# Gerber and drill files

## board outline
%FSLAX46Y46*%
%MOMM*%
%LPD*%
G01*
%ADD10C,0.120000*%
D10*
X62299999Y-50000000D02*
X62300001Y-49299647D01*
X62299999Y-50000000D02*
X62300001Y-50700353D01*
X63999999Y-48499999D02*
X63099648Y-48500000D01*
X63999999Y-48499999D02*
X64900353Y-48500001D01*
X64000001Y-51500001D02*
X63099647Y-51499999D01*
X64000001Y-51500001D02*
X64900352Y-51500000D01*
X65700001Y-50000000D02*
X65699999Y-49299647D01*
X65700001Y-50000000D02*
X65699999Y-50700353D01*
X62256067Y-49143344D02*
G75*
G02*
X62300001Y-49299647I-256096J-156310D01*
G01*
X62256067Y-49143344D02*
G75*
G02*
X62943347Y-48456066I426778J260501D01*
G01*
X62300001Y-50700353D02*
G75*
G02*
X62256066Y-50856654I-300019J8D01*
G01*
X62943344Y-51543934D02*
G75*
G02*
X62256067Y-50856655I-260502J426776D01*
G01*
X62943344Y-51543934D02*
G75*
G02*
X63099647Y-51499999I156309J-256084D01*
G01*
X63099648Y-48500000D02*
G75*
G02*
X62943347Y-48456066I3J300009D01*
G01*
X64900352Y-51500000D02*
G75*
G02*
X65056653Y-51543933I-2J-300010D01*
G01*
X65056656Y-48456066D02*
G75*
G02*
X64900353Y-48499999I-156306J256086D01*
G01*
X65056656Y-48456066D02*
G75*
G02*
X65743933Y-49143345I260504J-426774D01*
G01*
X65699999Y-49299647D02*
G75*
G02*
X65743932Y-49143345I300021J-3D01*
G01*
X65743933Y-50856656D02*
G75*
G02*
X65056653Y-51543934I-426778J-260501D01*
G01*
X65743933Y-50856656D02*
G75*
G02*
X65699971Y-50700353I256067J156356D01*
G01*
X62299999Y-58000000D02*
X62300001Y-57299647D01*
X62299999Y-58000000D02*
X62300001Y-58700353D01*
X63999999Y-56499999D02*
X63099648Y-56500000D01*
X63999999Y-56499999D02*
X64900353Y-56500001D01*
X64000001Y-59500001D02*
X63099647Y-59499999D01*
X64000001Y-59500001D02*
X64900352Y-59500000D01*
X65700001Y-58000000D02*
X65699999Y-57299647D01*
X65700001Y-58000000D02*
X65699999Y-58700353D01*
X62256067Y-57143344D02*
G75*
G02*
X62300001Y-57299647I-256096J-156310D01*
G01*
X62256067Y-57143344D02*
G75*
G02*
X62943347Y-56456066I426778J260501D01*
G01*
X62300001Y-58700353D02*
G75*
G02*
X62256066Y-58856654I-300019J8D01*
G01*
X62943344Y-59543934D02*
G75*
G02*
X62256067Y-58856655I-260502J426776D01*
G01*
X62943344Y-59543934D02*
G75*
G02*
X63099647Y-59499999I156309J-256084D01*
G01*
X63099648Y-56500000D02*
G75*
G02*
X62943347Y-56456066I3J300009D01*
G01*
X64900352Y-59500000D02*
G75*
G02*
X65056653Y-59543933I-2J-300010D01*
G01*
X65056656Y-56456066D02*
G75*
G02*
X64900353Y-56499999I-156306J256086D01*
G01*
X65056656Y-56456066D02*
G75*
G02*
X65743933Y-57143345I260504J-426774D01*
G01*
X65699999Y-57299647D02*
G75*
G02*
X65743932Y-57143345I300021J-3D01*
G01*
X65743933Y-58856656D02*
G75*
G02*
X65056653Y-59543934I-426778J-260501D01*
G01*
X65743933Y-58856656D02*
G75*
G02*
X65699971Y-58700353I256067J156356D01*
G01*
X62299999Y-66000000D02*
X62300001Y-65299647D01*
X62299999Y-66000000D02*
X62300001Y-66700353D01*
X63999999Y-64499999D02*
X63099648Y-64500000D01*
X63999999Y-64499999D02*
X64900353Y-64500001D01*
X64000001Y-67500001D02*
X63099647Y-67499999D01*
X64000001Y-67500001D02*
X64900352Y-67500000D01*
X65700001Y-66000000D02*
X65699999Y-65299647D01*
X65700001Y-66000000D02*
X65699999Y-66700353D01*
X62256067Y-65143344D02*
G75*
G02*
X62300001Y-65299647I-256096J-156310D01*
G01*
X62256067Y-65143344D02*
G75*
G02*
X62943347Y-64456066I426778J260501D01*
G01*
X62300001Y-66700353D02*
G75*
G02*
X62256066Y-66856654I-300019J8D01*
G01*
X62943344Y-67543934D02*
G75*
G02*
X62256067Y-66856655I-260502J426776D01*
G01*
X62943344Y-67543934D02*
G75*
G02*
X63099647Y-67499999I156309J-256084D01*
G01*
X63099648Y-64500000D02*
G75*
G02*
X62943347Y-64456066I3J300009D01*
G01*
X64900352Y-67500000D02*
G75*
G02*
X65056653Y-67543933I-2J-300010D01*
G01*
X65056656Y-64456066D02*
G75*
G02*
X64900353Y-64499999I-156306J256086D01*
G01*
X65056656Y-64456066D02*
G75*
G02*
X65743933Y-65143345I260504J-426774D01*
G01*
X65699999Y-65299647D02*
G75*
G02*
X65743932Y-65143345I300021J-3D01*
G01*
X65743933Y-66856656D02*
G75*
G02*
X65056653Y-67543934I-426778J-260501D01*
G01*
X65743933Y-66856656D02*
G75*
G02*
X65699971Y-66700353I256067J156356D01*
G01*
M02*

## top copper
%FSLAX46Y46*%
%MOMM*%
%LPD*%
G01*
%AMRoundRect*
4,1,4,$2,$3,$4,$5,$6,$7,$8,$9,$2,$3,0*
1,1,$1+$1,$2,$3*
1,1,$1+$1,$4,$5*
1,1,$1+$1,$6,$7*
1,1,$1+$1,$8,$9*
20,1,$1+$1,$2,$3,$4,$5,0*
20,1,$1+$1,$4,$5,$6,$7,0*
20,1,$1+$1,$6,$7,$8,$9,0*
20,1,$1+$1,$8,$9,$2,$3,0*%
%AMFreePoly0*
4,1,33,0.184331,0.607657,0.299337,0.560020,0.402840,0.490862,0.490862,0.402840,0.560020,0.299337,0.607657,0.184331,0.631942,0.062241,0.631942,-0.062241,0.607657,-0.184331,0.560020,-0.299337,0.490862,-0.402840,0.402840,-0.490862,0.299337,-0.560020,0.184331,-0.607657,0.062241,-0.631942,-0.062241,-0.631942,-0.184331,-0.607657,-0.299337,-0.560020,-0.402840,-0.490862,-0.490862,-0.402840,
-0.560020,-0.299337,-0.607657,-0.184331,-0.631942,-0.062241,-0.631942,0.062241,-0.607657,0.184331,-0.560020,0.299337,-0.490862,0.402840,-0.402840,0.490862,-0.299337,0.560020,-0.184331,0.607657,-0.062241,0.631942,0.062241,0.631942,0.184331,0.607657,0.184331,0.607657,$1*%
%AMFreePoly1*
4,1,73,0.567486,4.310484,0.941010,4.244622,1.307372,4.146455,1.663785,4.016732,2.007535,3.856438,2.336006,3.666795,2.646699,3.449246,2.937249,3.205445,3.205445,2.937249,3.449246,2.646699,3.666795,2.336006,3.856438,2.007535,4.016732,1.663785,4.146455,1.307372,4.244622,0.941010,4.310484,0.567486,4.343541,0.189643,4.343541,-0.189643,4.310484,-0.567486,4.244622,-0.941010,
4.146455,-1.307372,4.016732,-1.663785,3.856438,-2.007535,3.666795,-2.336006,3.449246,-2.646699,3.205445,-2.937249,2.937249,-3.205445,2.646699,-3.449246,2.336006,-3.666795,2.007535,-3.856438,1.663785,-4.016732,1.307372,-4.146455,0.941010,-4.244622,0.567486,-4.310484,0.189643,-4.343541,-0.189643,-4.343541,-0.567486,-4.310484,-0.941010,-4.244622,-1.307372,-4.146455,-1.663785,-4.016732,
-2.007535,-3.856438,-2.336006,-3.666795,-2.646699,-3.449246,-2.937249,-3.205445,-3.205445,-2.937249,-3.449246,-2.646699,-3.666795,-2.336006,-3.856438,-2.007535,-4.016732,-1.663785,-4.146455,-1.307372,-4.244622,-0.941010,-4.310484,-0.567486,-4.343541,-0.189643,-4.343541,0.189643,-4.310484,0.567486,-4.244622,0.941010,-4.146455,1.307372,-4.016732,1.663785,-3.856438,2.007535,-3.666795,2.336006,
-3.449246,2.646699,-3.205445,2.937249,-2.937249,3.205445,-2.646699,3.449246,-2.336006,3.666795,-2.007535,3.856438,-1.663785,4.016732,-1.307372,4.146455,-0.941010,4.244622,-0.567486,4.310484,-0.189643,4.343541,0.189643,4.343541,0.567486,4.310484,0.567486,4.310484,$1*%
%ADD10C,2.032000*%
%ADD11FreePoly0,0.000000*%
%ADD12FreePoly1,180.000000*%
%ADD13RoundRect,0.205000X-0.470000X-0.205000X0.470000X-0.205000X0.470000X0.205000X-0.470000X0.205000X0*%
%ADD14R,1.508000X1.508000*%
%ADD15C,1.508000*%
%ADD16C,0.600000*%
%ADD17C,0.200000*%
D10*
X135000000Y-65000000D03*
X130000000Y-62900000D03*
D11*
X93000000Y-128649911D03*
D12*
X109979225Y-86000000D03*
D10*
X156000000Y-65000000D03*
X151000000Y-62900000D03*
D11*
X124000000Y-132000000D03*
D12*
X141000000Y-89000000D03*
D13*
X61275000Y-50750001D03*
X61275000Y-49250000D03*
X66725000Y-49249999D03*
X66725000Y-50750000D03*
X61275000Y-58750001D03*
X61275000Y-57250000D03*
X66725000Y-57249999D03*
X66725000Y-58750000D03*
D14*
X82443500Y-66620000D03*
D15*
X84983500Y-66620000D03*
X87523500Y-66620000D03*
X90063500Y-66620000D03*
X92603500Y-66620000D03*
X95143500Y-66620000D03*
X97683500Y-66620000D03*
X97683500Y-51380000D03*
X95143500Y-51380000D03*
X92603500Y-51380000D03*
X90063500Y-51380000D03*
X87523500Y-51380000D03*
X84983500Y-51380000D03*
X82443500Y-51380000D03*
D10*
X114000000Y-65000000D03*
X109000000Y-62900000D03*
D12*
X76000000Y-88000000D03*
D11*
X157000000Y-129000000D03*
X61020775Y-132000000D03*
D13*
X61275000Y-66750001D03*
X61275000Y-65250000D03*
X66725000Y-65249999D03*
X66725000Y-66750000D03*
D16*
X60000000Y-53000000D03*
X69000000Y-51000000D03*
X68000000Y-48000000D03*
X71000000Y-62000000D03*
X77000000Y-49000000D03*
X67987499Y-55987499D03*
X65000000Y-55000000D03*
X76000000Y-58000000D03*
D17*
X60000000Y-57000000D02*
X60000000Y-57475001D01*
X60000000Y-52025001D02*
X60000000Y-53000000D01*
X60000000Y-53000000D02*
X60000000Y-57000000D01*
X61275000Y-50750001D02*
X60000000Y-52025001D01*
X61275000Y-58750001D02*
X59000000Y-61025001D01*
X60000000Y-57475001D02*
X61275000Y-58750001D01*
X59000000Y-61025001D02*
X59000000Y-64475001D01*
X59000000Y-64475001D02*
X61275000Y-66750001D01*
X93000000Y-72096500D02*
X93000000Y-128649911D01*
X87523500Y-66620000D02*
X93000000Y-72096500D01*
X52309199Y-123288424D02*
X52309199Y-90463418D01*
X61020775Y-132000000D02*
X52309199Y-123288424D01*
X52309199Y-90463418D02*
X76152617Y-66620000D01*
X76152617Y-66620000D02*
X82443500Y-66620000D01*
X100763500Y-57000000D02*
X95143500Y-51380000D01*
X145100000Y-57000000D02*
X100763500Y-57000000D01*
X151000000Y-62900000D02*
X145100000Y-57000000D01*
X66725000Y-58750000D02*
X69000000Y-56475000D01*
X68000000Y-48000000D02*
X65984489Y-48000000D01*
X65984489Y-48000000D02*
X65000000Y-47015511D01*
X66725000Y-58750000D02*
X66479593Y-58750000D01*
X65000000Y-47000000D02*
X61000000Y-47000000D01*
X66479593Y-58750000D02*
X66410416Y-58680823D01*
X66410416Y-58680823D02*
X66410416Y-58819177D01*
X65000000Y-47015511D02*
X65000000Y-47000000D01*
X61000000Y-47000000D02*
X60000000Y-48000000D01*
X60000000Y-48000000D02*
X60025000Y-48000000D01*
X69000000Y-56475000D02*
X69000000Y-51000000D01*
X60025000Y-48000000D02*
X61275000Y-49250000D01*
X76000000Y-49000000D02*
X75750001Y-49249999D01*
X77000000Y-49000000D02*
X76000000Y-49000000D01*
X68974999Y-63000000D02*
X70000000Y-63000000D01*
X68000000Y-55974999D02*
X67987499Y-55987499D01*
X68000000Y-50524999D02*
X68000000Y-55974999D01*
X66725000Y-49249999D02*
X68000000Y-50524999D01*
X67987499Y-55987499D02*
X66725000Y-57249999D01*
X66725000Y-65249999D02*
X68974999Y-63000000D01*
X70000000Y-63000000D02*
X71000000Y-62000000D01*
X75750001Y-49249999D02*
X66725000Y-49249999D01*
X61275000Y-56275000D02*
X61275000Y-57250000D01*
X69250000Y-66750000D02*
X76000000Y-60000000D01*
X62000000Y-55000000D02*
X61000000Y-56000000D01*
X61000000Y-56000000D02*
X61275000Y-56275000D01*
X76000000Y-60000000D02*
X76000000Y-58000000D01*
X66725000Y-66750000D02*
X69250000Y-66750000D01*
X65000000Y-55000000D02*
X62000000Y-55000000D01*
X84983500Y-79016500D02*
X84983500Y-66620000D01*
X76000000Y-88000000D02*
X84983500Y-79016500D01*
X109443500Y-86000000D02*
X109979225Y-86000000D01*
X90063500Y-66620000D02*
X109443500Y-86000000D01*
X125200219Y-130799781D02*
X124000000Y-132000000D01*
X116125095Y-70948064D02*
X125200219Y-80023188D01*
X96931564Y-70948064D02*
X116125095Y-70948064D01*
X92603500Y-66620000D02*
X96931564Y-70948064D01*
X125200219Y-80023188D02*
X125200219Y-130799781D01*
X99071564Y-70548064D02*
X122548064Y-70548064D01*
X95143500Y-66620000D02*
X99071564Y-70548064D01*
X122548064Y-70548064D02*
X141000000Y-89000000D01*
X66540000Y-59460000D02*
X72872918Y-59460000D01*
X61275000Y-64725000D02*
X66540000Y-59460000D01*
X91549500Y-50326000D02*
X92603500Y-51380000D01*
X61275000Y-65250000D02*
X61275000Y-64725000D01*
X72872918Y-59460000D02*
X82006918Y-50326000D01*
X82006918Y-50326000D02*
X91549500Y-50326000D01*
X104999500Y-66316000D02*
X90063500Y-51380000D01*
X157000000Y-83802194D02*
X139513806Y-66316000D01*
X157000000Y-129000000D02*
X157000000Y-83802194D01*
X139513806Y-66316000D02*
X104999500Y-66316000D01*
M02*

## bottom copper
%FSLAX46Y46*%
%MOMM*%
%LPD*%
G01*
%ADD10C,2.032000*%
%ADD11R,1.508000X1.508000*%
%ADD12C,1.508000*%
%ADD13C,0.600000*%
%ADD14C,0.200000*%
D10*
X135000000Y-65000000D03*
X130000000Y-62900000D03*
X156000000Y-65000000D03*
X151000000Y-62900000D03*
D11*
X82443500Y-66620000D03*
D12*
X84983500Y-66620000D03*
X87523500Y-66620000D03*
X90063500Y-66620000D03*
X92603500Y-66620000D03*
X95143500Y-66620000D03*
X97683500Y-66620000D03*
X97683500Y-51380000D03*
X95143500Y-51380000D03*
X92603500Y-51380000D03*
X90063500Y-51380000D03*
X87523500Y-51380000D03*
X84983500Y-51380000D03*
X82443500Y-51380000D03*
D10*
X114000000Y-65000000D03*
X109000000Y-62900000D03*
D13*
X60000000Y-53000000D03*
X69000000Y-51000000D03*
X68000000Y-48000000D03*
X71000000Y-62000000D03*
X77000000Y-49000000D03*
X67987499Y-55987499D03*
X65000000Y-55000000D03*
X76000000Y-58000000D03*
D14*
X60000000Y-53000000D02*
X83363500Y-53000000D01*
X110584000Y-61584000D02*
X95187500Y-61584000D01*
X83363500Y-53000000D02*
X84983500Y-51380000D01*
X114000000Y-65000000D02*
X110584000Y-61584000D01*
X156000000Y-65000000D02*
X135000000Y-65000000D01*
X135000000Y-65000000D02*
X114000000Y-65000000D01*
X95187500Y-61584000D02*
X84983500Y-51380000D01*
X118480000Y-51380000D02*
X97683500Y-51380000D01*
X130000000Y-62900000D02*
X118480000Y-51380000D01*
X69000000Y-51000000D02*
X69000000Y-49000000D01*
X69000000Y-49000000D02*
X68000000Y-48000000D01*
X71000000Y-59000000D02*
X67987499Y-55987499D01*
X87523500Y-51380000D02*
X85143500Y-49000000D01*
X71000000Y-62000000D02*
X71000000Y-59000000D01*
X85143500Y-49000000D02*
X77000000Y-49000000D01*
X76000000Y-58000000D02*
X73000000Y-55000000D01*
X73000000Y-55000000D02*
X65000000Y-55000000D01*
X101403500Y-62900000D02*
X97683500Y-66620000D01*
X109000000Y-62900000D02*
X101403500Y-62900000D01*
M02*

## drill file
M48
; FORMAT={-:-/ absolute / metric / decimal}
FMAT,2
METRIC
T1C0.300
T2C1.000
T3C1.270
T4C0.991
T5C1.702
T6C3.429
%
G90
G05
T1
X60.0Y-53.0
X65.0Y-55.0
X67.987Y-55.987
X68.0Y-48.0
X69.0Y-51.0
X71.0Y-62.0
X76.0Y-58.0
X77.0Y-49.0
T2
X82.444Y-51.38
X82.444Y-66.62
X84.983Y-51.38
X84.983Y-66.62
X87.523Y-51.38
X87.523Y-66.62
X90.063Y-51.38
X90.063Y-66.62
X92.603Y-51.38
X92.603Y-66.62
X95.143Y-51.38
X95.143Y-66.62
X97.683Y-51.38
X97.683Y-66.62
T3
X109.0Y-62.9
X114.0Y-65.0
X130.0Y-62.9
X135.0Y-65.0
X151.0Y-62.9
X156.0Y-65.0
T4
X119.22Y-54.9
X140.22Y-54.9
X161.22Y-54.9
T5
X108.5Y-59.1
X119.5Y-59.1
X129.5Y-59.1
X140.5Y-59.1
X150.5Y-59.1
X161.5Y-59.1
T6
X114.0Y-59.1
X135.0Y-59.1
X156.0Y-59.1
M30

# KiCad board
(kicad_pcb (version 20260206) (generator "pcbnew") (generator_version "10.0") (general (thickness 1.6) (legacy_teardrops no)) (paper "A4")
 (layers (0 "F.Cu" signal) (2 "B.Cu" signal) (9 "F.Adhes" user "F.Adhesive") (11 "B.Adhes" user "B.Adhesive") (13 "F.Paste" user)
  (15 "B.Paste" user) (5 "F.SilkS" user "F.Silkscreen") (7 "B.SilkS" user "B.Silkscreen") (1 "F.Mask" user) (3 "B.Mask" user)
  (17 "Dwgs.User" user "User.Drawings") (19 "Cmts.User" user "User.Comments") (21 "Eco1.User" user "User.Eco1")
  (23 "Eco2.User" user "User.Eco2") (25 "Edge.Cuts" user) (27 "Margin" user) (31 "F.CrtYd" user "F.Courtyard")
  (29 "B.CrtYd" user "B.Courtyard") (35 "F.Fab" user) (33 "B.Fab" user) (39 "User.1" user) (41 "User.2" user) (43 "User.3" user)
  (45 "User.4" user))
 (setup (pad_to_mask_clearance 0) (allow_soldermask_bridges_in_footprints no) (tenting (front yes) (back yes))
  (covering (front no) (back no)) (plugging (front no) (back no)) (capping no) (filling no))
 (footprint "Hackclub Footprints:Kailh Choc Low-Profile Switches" (layer "F.Cu") (at 135 59.100001)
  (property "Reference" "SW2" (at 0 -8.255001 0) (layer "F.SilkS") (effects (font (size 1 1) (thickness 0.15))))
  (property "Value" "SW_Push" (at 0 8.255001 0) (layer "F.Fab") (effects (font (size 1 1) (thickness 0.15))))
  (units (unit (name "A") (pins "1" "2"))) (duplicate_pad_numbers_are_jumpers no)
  (pad "" np_thru_hole circle (at -5.5 0) (size 1.7018 1.7018) (drill 1.7018) (layers "*.Cu" "*.Mask"))
  (pad "" np_thru_hole circle (at 0 0) (size 3.429 3.429) (drill 3.429) (layers "*.Cu" "*.Mask"))
  (pad "" np_thru_hole circle (at 5.22 -4.2) (size 0.9906 0.9906) (drill 0.9906) (layers "*.Cu" "*.Mask"))
  (pad "" np_thru_hole circle (at 5.5 0) (size 1.7018 1.7018) (drill 1.7018) (layers "*.Cu" "*.Mask"))
  (pad "1" thru_hole circle (at 0 5.899999) (size 2.032 2.032) (drill 1.27) (layers "*.Cu" "*.Mask") (remove_unused_layers no) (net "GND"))
  (pad "2" thru_hole circle (at -5 3.799999) (size 2.032 2.032) (drill 1.27) (layers "*.Cu" "*.Mask") (remove_unused_layers no)
   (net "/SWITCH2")))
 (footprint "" (layer "F.Cu") (at 93 128.649911)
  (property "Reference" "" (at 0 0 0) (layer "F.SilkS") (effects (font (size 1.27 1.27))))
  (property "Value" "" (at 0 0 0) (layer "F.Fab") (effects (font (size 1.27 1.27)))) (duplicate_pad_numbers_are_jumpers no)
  (pad "3" smd custom (at 0 0) (size 1.27 1.27) (layers "F.Cu" "F.Mask") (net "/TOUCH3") (thermal_bridge_angle 90)
   (options (clearance outline) (anchor circle)) (primitives)))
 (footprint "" (layer "F.Cu") (at 109.979225 86)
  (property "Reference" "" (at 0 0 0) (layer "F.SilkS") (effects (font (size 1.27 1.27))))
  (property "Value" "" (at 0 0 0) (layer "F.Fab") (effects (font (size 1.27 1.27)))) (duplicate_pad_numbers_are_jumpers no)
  (pad "4" smd custom (at 0 0 180) (size 8.695358 8.695358) (layers "F.Cu" "F.Mask") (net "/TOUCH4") (thermal_bridge_angle 90)
   (options (clearance outline) (anchor circle)) (primitives)))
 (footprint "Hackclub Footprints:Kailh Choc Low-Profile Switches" (layer "F.Cu") (at 156 59.100001)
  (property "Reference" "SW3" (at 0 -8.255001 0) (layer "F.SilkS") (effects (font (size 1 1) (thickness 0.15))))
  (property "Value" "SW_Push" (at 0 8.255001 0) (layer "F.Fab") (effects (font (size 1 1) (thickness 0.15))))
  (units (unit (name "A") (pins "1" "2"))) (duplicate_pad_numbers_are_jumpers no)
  (pad "" np_thru_hole circle (at -5.5 0) (size 1.7018 1.7018) (drill 1.7018) (layers "*.Cu" "*.Mask"))
  (pad "" np_thru_hole circle (at 0 0) (size 3.429 3.429) (drill 3.429) (layers "*.Cu" "*.Mask"))
  (pad "" np_thru_hole circle (at 5.22 -4.2) (size 0.9906 0.9906) (drill 0.9906) (layers "*.Cu" "*.Mask"))
  (pad "" np_thru_hole circle (at 5.5 0) (size 1.7018 1.7018) (drill 1.7018) (layers "*.Cu" "*.Mask"))
  (pad "1" thru_hole circle (at 0 5.899999) (size 2.032 2.032) (drill 1.27) (layers "*.Cu" "*.Mask") (remove_unused_layers no) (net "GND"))
  (pad "2" thru_hole circle (at -5 3.799999) (size 2.032 2.032) (drill 1.27) (layers "*.Cu" "*.Mask") (remove_unused_layers no)
   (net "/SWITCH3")))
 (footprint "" (layer "F.Cu") (at 124 132)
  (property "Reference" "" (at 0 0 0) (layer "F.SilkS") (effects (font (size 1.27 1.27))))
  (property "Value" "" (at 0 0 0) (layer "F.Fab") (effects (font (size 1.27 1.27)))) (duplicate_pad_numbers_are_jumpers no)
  (pad "5" smd custom (at 0 0) (size 1.27 1.27) (layers "F.Cu" "F.Mask") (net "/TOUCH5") (thermal_bridge_angle 90)
   (options (clearance outline) (anchor circle)) (primitives)))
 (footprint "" (layer "F.Cu") (at 141 89)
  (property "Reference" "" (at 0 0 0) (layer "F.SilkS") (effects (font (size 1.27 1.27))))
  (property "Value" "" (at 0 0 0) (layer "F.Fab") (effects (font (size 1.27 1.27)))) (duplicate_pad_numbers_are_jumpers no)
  (pad "6" smd custom (at 0 0 180) (size 8.695358 8.695358) (layers "F.Cu" "F.Mask") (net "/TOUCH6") (thermal_bridge_angle 90)
   (options (clearance outline) (anchor circle)) (primitives)))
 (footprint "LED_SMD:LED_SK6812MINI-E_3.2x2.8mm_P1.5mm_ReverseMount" (layer "F.Cu") (at 64 50)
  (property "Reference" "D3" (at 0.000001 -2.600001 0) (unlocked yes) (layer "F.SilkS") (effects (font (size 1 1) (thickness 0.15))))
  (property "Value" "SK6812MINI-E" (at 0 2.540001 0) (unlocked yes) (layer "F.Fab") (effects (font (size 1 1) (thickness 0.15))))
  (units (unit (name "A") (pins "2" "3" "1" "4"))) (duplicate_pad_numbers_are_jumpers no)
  (fp_line (start -1.700001 0) (end -1.699999 -0.700353) (stroke (width 0.12) (type solid)) (layer "Edge.Cuts"))
  (fp_line (start -1.700001 0) (end -1.699999 0.700353) (stroke (width 0.12) (type solid)) (layer "Edge.Cuts"))
  (fp_line (start -0.000001 -1.500001) (end -0.900352 -1.5) (stroke (width 0.12) (type solid)) (layer "Edge.Cuts"))
  (fp_line (start -0.000001 -1.500001) (end 0.900353 -1.499999) (stroke (width 0.12) (type solid)) (layer "Edge.Cuts"))
  (fp_line (start 0.000001 1.500001) (end -0.900353 1.499999) (stroke (width 0.12) (type solid)) (layer "Edge.Cuts"))
  (fp_line (start 0.000001 1.500001) (end 0.900352 1.5) (stroke (width 0.12) (type solid)) (layer "Edge.Cuts"))
  (fp_line (start 1.700001 0) (end 1.699999 -0.700353) (stroke (width 0.12) (type solid)) (layer "Edge.Cuts"))
  (fp_line (start 1.700001 0) (end 1.699999 0.700353) (stroke (width 0.12) (type solid)) (layer "Edge.Cuts"))
  (fp_arc (start -1.743933 -0.856656) (mid -1.711192 -0.781532) (end -1.699999 -0.700353) (stroke (width 0.12) (type solid))
   (layer "Edge.Cuts"))
  (fp_arc (start -1.743933 -0.856656) (mid -1.670709 -1.47071) (end -1.056653 -1.543934) (stroke (width 0.12) (type solid))
   (layer "Edge.Cuts"))
  (fp_arc (start -1.699999 0.700353) (mid -1.711192 0.78153) (end -1.743934 0.856654) (stroke (width 0.12) (type solid)) (layer "Edge.Cuts"))
  (fp_arc (start -1.056656 1.543934) (mid -1.670711 1.470711) (end -1.743934 0.856654) (stroke (width 0.12) (type solid))
   (layer "Edge.Cuts"))
  (fp_arc (start -1.056656 1.543934) (mid -0.981532 1.511192) (end -0.900353 1.499999) (stroke (width 0.12) (type solid))
   (layer "Edge.Cuts"))
  (fp_arc (start -0.900352 -1.5) (mid -0.981532 -1.511193) (end -1.056653 -1.543934) (stroke (width 0.12) (type solid)) (layer "Edge.Cuts"))
  (fp_arc (start 0.900352 1.5) (mid 0.981532 1.511193) (end 1.056653 1.543934) (stroke (width 0.12) (type solid)) (layer "Edge.Cuts"))
  (fp_arc (start 1.056656 -1.543934) (mid 0.981532 -1.511192) (end 0.900353 -1.499999) (stroke (width 0.12) (type solid))
   (layer "Edge.Cuts"))
  (fp_arc (start 1.056656 -1.543934) (mid 1.670711 -1.470711) (end 1.743934 -0.856654) (stroke (width 0.12) (type solid))
   (layer "Edge.Cuts"))
  (fp_arc (start 1.699999 -0.700353) (mid 1.711192 -0.78153) (end 1.743934 -0.856654) (stroke (width 0.12) (type solid)) (layer "Edge.Cuts"))
  (fp_arc (start 1.743933 0.856656) (mid 1.670709 1.47071) (end 1.056653 1.543934) (stroke (width 0.12) (type solid)) (layer "Edge.Cuts"))
  (fp_arc (start 1.743933 0.856656) (mid 1.711192 0.781532) (end 1.699999 0.700353) (stroke (width 0.12) (type solid)) (layer "Edge.Cuts"))
  (pad "1" smd roundrect (at -2.725 0.750001) (size 1.35 0.82) (layers "F.Cu" "F.Mask" "F.Paste") (roundrect_rratio 0.25) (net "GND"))
  (pad "2" smd roundrect (at -2.725 -0.75) (size 1.35 0.82) (layers "F.Cu" "F.Mask" "F.Paste") (roundrect_rratio 0.25) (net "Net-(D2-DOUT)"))
  (pad "3" smd roundrect (at 2.725 -0.750001) (size 1.35 0.82) (layers "F.Cu" "F.Mask" "F.Paste") (roundrect_rratio 0.25) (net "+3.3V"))
  (pad "4" smd roundrect (at 2.725 0.75) (size 1.35 0.82) (layers "F.Cu" "F.Mask" "F.Paste") (roundrect_rratio 0.25)
   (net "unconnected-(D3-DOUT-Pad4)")))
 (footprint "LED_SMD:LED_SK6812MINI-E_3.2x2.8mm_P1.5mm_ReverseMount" (layer "F.Cu") (at 64 58)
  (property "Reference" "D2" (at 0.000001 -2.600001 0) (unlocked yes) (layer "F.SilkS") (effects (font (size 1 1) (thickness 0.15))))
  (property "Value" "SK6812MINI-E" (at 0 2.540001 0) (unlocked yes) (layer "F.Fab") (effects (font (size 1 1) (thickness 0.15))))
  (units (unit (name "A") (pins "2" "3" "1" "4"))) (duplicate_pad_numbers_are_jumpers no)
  (fp_line (start -1.700001 0) (end -1.699999 -0.700353) (stroke (width 0.12) (type solid)) (layer "Edge.Cuts"))
  (fp_line (start -1.700001 0) (end -1.699999 0.700353) (stroke (width 0.12) (type solid)) (layer "Edge.Cuts"))
  (fp_line (start -0.000001 -1.500001) (end -0.900352 -1.5) (stroke (width 0.12) (type solid)) (layer "Edge.Cuts"))
  (fp_line (start -0.000001 -1.500001) (end 0.900353 -1.499999) (stroke (width 0.12) (type solid)) (layer "Edge.Cuts"))
  (fp_line (start 0.000001 1.500001) (end -0.900353 1.499999) (stroke (width 0.12) (type solid)) (layer "Edge.Cuts"))
  (fp_line (start 0.000001 1.500001) (end 0.900352 1.5) (stroke (width 0.12) (type solid)) (layer "Edge.Cuts"))
  (fp_line (start 1.700001 0) (end 1.699999 -0.700353) (stroke (width 0.12) (type solid)) (layer "Edge.Cuts"))
  (fp_line (start 1.700001 0) (end 1.699999 0.700353) (stroke (width 0.12) (type solid)) (layer "Edge.Cuts"))
  (fp_arc (start -1.743933 -0.856656) (mid -1.711192 -0.781532) (end -1.699999 -0.700353) (stroke (width 0.12) (type solid))
   (layer "Edge.Cuts"))
  (fp_arc (start -1.743933 -0.856656) (mid -1.670709 -1.47071) (end -1.056653 -1.543934) (stroke (width 0.12) (type solid))
   (layer "Edge.Cuts"))
  (fp_arc (start -1.699999 0.700353) (mid -1.711192 0.78153) (end -1.743934 0.856654) (stroke (width 0.12) (type solid)) (layer "Edge.Cuts"))
  (fp_arc (start -1.056656 1.543934) (mid -1.670711 1.470711) (end -1.743934 0.856654) (stroke (width 0.12) (type solid))
   (layer "Edge.Cuts"))
  (fp_arc (start -1.056656 1.543934) (mid -0.981532 1.511192) (end -0.900353 1.499999) (stroke (width 0.12) (type solid))
   (layer "Edge.Cuts"))
  (fp_arc (start -0.900352 -1.5) (mid -0.981532 -1.511193) (end -1.056653 -1.543934) (stroke (width 0.12) (type solid)) (layer "Edge.Cuts"))
  (fp_arc (start 0.900352 1.5) (mid 0.981532 1.511193) (end 1.056653 1.543934) (stroke (width 0.12) (type solid)) (layer "Edge.Cuts"))
  (fp_arc (start 1.056656 -1.543934) (mid 0.981532 -1.511192) (end 0.900353 -1.499999) (stroke (width 0.12) (type solid))
   (layer "Edge.Cuts"))
  (fp_arc (start 1.056656 -1.543934) (mid 1.670711 -1.470711) (end 1.743934 -0.856654) (stroke (width 0.12) (type solid))
   (layer "Edge.Cuts"))
  (fp_arc (start 1.699999 -0.700353) (mid 1.711192 -0.78153) (end 1.743934 -0.856654) (stroke (width 0.12) (type solid)) (layer "Edge.Cuts"))
  (fp_arc (start 1.743933 0.856656) (mid 1.670709 1.47071) (end 1.056653 1.543934) (stroke (width 0.12) (type solid)) (layer "Edge.Cuts"))
  (fp_arc (start 1.743933 0.856656) (mid 1.711192 0.781532) (end 1.699999 0.700353) (stroke (width 0.12) (type solid)) (layer "Edge.Cuts"))
  (pad "1" smd roundrect (at -2.725 0.750001) (size 1.35 0.82) (layers "F.Cu" "F.Mask" "F.Paste") (roundrect_rratio 0.25) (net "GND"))
  (pad "2" smd roundrect (at -2.725 -0.75) (size 1.35 0.82) (layers "F.Cu" "F.Mask" "F.Paste") (roundrect_rratio 0.25) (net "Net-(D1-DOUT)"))
  (pad "3" smd roundrect (at 2.725 -0.750001) (size 1.35 0.82) (layers "F.Cu" "F.Mask" "F.Paste") (roundrect_rratio 0.25) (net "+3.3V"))
  (pad "4" smd roundrect (at 2.725 0.75) (size 1.35 0.82) (layers "F.Cu" "F.Mask" "F.Paste") (roundrect_rratio 0.25) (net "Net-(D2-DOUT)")))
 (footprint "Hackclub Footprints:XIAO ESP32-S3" (layer "F.Cu") (at 90 59 90)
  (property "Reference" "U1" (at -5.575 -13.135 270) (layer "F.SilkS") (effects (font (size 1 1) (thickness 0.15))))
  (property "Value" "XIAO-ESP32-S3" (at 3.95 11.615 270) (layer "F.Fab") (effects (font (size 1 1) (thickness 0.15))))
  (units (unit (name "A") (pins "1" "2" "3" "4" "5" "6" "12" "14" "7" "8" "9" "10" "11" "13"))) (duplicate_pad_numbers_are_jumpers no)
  (pad "1" thru_hole rect (at -7.62 -7.5565 90) (size 1.508 1.508) (drill 1) (layers "*.Cu" "*.Mask") (remove_unused_layers no)
   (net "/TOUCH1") (solder_mask_margin 0.102))
  (pad "2" thru_hole circle (at -7.62 -5.0165 90) (size 1.508 1.508) (drill 1) (layers "*.Cu" "*.Mask") (remove_unused_layers no)
   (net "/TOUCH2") (solder_mask_margin 0.102))
  (pad "3" thru_hole circle (at -7.62 -2.4765 90) (size 1.508 1.508) (drill 1) (layers "*.Cu" "*.Mask") (remove_unused_layers no)
   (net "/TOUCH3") (solder_mask_margin 0.102))
  (pad "4" thru_hole circle (at -7.62 0.0635 90) (size 1.508 1.508) (drill 1) (layers "*.Cu" "*.Mask") (remove_unused_layers no)
   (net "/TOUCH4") (solder_mask_margin 0.102))
  (pad "5" thru_hole circle (at -7.62 2.6035 90) (size 1.508 1.508) (drill 1) (layers "*.Cu" "*.Mask") (remove_unused_layers no)
   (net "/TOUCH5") (solder_mask_margin 0.102))
  (pad "6" thru_hole circle (at -7.62 5.1435 90) (size 1.508 1.508) (drill 1) (layers "*.Cu" "*.Mask") (remove_unused_layers no)
   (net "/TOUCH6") (solder_mask_margin 0.102))
  (pad "7" thru_hole circle (at -7.62 7.6835 90) (size 1.508 1.508) (drill 1) (layers "*.Cu" "*.Mask") (remove_unused_layers no)
   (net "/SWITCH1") (solder_mask_margin 0.102))
  (pad "8" thru_hole circle (at 7.62 7.6835 90) (size 1.508 1.508) (drill 1) (layers "*.Cu" "*.Mask") (remove_unused_layers no)
   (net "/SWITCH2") (solder_mask_margin 0.102))
  (pad "9" thru_hole circle (at 7.62 5.1435 90) (size 1.508 1.508) (drill 1) (layers "*.Cu" "*.Mask") (remove_unused_layers no)
   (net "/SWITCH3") (solder_mask_margin 0.102))
  (pad "10" thru_hole circle (at 7.62 2.6035 90) (size 1.508 1.508) (drill 1) (layers "*.Cu" "*.Mask") (remove_unused_layers no)
   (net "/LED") (solder_mask_margin 0.102))
  (pad "11" thru_hole circle (at 7.62 0.0635 90) (size 1.508 1.508) (drill 1) (layers "*.Cu" "*.Mask") (remove_unused_layers no)
   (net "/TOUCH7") (solder_mask_margin 0.102))
  (pad "12" thru_hole circle (at 7.62 -2.4765 90) (size 1.508 1.508) (drill 1) (layers "*.Cu" "*.Mask") (remove_unused_layers no)
   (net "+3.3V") (solder_mask_margin 0.102))
  (pad "13" thru_hole circle (at 7.62 -5.0165 90) (size 1.508 1.508) (drill 1) (layers "*.Cu" "*.Mask") (remove_unused_layers no)
   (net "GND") (solder_mask_margin 0.102))
  (pad "14" thru_hole circle (at 7.62 -7.5565 90) (size 1.508 1.508) (drill 1) (layers "*.Cu" "*.Mask") (remove_unused_layers no)
   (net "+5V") (solder_mask_margin 0.102)))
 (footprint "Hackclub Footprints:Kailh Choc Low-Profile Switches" (layer "F.Cu") (at 114 59.100001)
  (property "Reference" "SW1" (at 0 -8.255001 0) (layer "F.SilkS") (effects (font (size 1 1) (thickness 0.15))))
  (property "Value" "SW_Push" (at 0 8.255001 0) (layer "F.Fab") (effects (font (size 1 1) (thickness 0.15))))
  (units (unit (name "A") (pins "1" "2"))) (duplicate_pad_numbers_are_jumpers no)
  (pad "" np_thru_hole circle (at -5.5 0) (size 1.7018 1.7018) (drill 1.7018) (layers "*.Cu" "*.Mask"))
  (pad "" np_thru_hole circle (at 0 0) (size 3.429 3.429) (drill 3.429) (layers "*.Cu" "*.Mask"))
  (pad "" np_thru_hole circle (at 5.22 -4.2) (size 0.9906 0.9906) (drill 0.9906) (layers "*.Cu" "*.Mask"))
  (pad "" np_thru_hole circle (at 5.5 0) (size 1.7018 1.7018) (drill 1.7018) (layers "*.Cu" "*.Mask"))
  (pad "1" thru_hole circle (at 0 5.899999) (size 2.032 2.032) (drill 1.27) (layers "*.Cu" "*.Mask") (remove_unused_layers no) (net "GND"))
  (pad "2" thru_hole circle (at -5 3.799999) (size 2.032 2.032) (drill 1.27) (layers "*.Cu" "*.Mask") (remove_unused_layers no)
   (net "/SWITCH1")))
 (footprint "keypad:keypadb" (layer "F.Cu") (at 76 103.301057 180)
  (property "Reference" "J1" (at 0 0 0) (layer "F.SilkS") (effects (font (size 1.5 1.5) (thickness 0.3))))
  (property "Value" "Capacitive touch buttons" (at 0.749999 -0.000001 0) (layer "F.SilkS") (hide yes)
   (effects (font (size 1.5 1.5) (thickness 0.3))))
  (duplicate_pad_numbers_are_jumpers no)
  (pad "2" smd custom (at 0 15.301057 180) (size 8.695358 8.695358) (layers "F.Cu" "F.Mask") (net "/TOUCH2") (thermal_bridge_angle 90)
   (options (clearance outline) (anchor circle)) (primitives)))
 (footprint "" (layer "F.Cu") (at 157 129)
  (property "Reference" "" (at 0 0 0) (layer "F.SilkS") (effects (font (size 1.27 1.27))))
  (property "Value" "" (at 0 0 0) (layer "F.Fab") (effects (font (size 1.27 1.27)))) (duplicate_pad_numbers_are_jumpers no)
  (pad "7" smd custom (at 0 0) (size 1.27 1.27) (layers "F.Cu" "F.Mask") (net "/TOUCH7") (thermal_bridge_angle 90)
   (options (clearance outline) (anchor circle)) (primitives)))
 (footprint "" (layer "F.Cu") (at 61.020775 132)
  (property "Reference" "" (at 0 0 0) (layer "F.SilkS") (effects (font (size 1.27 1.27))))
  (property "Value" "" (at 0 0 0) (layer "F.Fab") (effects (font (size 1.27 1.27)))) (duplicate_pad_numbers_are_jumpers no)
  (pad "1" smd custom (at 0 0) (size 1.27 1.27) (layers "F.Cu" "F.Mask") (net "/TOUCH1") (thermal_bridge_angle 90)
   (options (clearance outline) (anchor circle)) (primitives)))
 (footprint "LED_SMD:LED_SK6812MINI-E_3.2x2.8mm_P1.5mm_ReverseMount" (layer "F.Cu") (at 64 66)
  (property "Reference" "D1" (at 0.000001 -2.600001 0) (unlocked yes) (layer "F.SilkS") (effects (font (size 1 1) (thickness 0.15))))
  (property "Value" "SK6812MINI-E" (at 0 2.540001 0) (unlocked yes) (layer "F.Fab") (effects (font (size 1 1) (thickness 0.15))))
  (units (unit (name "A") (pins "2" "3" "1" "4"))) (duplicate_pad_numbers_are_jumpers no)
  (fp_line (start -1.700001 0) (end -1.699999 -0.700353) (stroke (width 0.12) (type solid)) (layer "Edge.Cuts"))
  (fp_line (start -1.700001 0) (end -1.699999 0.700353) (stroke (width 0.12) (type solid)) (layer "Edge.Cuts"))
  (fp_line (start -0.000001 -1.500001) (end -0.900352 -1.5) (stroke (width 0.12) (type solid)) (layer "Edge.Cuts"))
  (fp_line (start -0.000001 -1.500001) (end 0.900353 -1.499999) (stroke (width 0.12) (type solid)) (layer "Edge.Cuts"))
  (fp_line (start 0.000001 1.500001) (end -0.900353 1.499999) (stroke (width 0.12) (type solid)) (layer "Edge.Cuts"))
  (fp_line (start 0.000001 1.500001) (end 0.900352 1.5) (stroke (width 0.12) (type solid)) (layer "Edge.Cuts"))
  (fp_line (start 1.700001 0) (end 1.699999 -0.700353) (stroke (width 0.12) (type solid)) (layer "Edge.Cuts"))
  (fp_line (start 1.700001 0) (end 1.699999 0.700353) (stroke (width 0.12) (type solid)) (layer "Edge.Cuts"))
  (fp_arc (start -1.743933 -0.856656) (mid -1.711192 -0.781532) (end -1.699999 -0.700353) (stroke (width 0.12) (type solid))
   (layer "Edge.Cuts"))
  (fp_arc (start -1.743933 -0.856656) (mid -1.670709 -1.47071) (end -1.056653 -1.543934) (stroke (width 0.12) (type solid))
   (layer "Edge.Cuts"))
  (fp_arc (start -1.699999 0.700353) (mid -1.711192 0.78153) (end -1.743934 0.856654) (stroke (width 0.12) (type solid)) (layer "Edge.Cuts"))
  (fp_arc (start -1.056656 1.543934) (mid -1.670711 1.470711) (end -1.743934 0.856654) (stroke (width 0.12) (type solid))
   (layer "Edge.Cuts"))
  (fp_arc (start -1.056656 1.543934) (mid -0.981532 1.511192) (end -0.900353 1.499999) (stroke (width 0.12) (type solid))
   (layer "Edge.Cuts"))
  (fp_arc (start -0.900352 -1.5) (mid -0.981532 -1.511193) (end -1.056653 -1.543934) (stroke (width 0.12) (type solid)) (layer "Edge.Cuts"))
  (fp_arc (start 0.900352 1.5) (mid 0.981532 1.511193) (end 1.056653 1.543934) (stroke (width 0.12) (type solid)) (layer "Edge.Cuts"))
  (fp_arc (start 1.056656 -1.543934) (mid 0.981532 -1.511192) (end 0.900353 -1.499999) (stroke (width 0.12) (type solid))
   (layer "Edge.Cuts"))
  (fp_arc (start 1.056656 -1.543934) (mid 1.670711 -1.470711) (end 1.743934 -0.856654) (stroke (width 0.12) (type solid))
   (layer "Edge.Cuts"))
  (fp_arc (start 1.699999 -0.700353) (mid 1.711192 -0.78153) (end 1.743934 -0.856654) (stroke (width 0.12) (type solid)) (layer "Edge.Cuts"))
  (fp_arc (start 1.743933 0.856656) (mid 1.670709 1.47071) (end 1.056653 1.543934) (stroke (width 0.12) (type solid)) (layer "Edge.Cuts"))
  (fp_arc (start 1.743933 0.856656) (mid 1.711192 0.781532) (end 1.699999 0.700353) (stroke (width 0.12) (type solid)) (layer "Edge.Cuts"))
  (pad "1" smd roundrect (at -2.725 0.750001) (size 1.35 0.82) (layers "F.Cu" "F.Mask" "F.Paste") (roundrect_rratio 0.25) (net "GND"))
  (pad "2" smd roundrect (at -2.725 -0.75) (size 1.35 0.82) (layers "F.Cu" "F.Mask" "F.Paste") (roundrect_rratio 0.25) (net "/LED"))
  (pad "3" smd roundrect (at 2.725 -0.750001) (size 1.35 0.82) (layers "F.Cu" "F.Mask" "F.Paste") (roundrect_rratio 0.25) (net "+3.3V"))
  (pad "4" smd roundrect (at 2.725 0.75) (size 1.35 0.82) (layers "F.Cu" "F.Mask" "F.Paste") (roundrect_rratio 0.25) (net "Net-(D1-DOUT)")))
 (segment (start 60 57) (end 60 57.475001) (width 0.2) (layer "F.Cu") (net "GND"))
 (segment (start 60 52.025001) (end 60 53) (width 0.2) (layer "F.Cu") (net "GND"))
 (segment (start 60 53) (end 60 57) (width 0.2) (layer "F.Cu") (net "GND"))
 (segment (start 61.275 50.750001) (end 60 52.025001) (width 0.2) (layer "F.Cu") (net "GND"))
 (segment (start 61.275 58.750001) (end 59 61.025001) (width 0.2) (layer "F.Cu") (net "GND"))
 (segment (start 60 57.475001) (end 61.275 58.750001) (width 0.2) (layer "F.Cu") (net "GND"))
 (segment (start 59 61.025001) (end 59 64.475001) (width 0.2) (layer "F.Cu") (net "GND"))
 (segment (start 59 64.475001) (end 61.275 66.750001) (width 0.2) (layer "F.Cu") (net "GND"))
 (via (at 60 53) (size 0.6) (drill 0.3) (layers "F.Cu" "B.Cu") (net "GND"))
 (segment (start 60 53) (end 83.3635 53) (width 0.2) (layer "B.Cu") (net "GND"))
 (segment (start 110.584 61.584) (end 95.1875 61.584) (width 0.2) (layer "B.Cu") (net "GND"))
 (segment (start 83.3635 53) (end 84.9835 51.38) (width 0.2) (layer "B.Cu") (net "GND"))
 (segment (start 114 65) (end 110.584 61.584) (width 0.2) (layer "B.Cu") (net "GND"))
 (segment (start 156 65) (end 135 65) (width 0.2) (layer "B.Cu") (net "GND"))
 (segment (start 135 65) (end 114 65) (width 0.2) (layer "B.Cu") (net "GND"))
 (segment (start 95.1875 61.584) (end 84.9835 51.38) (width 0.2) (layer "B.Cu") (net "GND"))
 (segment (start 118.48 51.38) (end 97.6835 51.38) (width 0.2) (layer "B.Cu") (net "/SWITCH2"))
 (segment (start 130 62.9) (end 118.48 51.38) (width 0.2) (layer "B.Cu") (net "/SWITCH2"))
 (segment (start 93 72.0965) (end 93 128.649911) (width 0.2) (layer "F.Cu") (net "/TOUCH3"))
 (segment (start 87.5235 66.62) (end 93 72.0965) (width 0.2) (layer "F.Cu") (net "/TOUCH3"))
 (segment (start 52.309199 123.288424) (end 52.309199 90.463418) (width 0.2) (layer "F.Cu") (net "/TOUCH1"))
 (segment (start 61.020775 132) (end 52.309199 123.288424) (width 0.2) (layer "F.Cu") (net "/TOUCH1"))
 (segment (start 52.309199 90.463418) (end 76.152617 66.62) (width 0.2) (layer "F.Cu") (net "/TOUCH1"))
 (segment (start 76.152617 66.62) (end 82.4435 66.62) (width 0.2) (layer "F.Cu") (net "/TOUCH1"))
 (segment (start 100.7635 57) (end 95.1435 51.38) (width 0.2) (layer "F.Cu") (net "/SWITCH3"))
 (segment (start 145.1 57) (end 100.7635 57) (width 0.2) (layer "F.Cu") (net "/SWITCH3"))
 (segment (start 151 62.9) (end 145.1 57) (width 0.2) (layer "F.Cu") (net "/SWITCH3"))
 (segment (start 66.725 58.75) (end 69 56.475) (width 0.2) (layer "F.Cu") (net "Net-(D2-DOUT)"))
 (segment (start 68 48) (end 65.984489 48) (width 0.2) (layer "F.Cu") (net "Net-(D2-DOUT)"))
 (segment (start 65.984489 48) (end 65 47.015511) (width 0.2) (layer "F.Cu") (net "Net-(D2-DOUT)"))
 (segment (start 66.725 58.75) (end 66.479593 58.75) (width 0.2) (layer "F.Cu") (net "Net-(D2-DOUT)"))
 (segment (start 65 47) (end 61 47) (width 0.2) (layer "F.Cu") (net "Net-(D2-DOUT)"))
 (segment (start 66.479593 58.75) (end 66.410416 58.680823) (width 0.2) (layer "F.Cu") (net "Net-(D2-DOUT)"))
 (segment (start 66.410416 58.680823) (end 66.410416 58.819177) (width 0.2) (layer "F.Cu") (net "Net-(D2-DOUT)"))
 (segment (start 65 47.015511) (end 65 47) (width 0.2) (layer "F.Cu") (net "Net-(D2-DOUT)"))
 (segment (start 61 47) (end 60 48) (width 0.2) (layer "F.Cu") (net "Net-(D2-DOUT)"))
 (segment (start 60 48) (end 60.025 48) (width 0.2) (layer "F.Cu") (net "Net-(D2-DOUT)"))
 (segment (start 69 56.475) (end 69 51) (width 0.2) (layer "F.Cu") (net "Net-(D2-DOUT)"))
 (segment (start 60.025 48) (end 61.275 49.25) (width 0.2) (layer "F.Cu") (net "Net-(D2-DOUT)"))
 (via (at 69 51) (size 0.6) (drill 0.3) (layers "F.Cu" "B.Cu") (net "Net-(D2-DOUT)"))
 (via (at 68 48) (size 0.6) (drill 0.3) (layers "F.Cu" "B.Cu") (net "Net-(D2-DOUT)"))
 (segment (start 69 51) (end 69 49) (width 0.2) (layer "B.Cu") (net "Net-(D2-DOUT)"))
 (segment (start 69 49) (end 68 48) (width 0.2) (layer "B.Cu") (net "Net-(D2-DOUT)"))
 (segment (start 76 49) (end 75.750001 49.249999) (width 0.2) (layer "F.Cu") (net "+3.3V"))
 (segment (start 77 49) (end 76 49) (width 0.2) (layer "F.Cu") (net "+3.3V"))
 (segment (start 68.974999 63) (end 70 63) (width 0.2) (layer "F.Cu") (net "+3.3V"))
 (segment (start 68 55.974999) (end 67.987499 55.987499) (width 0.2) (layer "F.Cu") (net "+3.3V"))
 (segment (start 68 50.524999) (end 68 55.974999) (width 0.2) (layer "F.Cu") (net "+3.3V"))
 (segment (start 66.725 49.249999) (end 68 50.524999) (width 0.2) (layer "F.Cu") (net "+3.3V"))
 (segment (start 67.987499 55.987499) (end 66.725 57.249999) (width 0.2) (layer "F.Cu") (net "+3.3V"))
 (segment (start 66.725 65.249999) (end 68.974999 63) (width 0.2) (layer "F.Cu") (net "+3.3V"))
 (segment (start 70 63) (end 71 62) (width 0.2) (layer "F.Cu") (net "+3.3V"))
 (segment (start 75.750001 49.249999) (end 66.725 49.249999) (width 0.2) (layer "F.Cu") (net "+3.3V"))
 (via (at 71 62) (size 0.6) (drill 0.3) (layers "F.Cu" "B.Cu") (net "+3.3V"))
 (via (at 77 49) (size 0.6) (drill 0.3) (layers "F.Cu" "B.Cu") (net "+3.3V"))
 (via (at 67.987499 55.987499) (size 0.6) (drill 0.3) (layers "F.Cu" "B.Cu") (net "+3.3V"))
 (segment (start 71 59) (end 67.987499 55.987499) (width 0.2) (layer "B.Cu") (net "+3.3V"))
 (segment (start 87.5235 51.38) (end 85.1435 49) (width 0.2) (layer "B.Cu") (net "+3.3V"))
 (segment (start 71 62) (end 71 59) (width 0.2) (layer "B.Cu") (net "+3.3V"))
 (segment (start 85.1435 49) (end 77 49) (width 0.2) (layer "B.Cu") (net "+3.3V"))
 (segment (start 61.275 56.275) (end 61.275 57.25) (width 0.2) (layer "F.Cu") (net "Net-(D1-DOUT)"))
 (segment (start 69.25 66.75) (end 76 60) (width 0.2) (layer "F.Cu") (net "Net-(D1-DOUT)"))
 (segment (start 62 55) (end 61 56) (width 0.2) (layer "F.Cu") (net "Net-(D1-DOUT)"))
 (segment (start 61 56) (end 61.275 56.275) (width 0.2) (layer "F.Cu") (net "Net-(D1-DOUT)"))
 (segment (start 76 60) (end 76 58) (width 0.2) (layer "F.Cu") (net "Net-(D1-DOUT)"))
 (segment (start 66.725 66.75) (end 69.25 66.75) (width 0.2) (layer "F.Cu") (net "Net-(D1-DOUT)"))
 (segment (start 65 55) (end 62 55) (width 0.2) (layer "F.Cu") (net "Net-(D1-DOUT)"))
 (via (at 65 55) (size 0.6) (drill 0.3) (layers "F.Cu" "B.Cu") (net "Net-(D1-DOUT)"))
 (via (at 76 58) (size 0.6) (drill 0.3) (layers "F.Cu" "B.Cu") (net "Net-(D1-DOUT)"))
 (segment (start 76 58) (end 73 55) (width 0.2) (layer "B.Cu") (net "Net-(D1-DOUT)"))
 (segment (start 73 55) (end 65 55) (width 0.2) (layer "B.Cu") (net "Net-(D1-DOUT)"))
 (segment (start 84.9835 79.0165) (end 84.9835 66.62) (width 0.2) (layer "F.Cu") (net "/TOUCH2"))
 (segment (start 76 88) (end 84.9835 79.0165) (width 0.2) (layer "F.Cu") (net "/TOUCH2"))
 (segment (start 109.4435 86) (end 109.979225 86) (width 0.2) (layer "F.Cu") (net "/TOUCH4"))
 (segment (start 90.0635 66.62) (end 109.4435 86) (width 0.2) (layer "F.Cu") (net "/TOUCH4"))
 (segment (start 125.200219 130.799781) (end 124 132) (width 0.2) (layer "F.Cu") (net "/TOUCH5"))
 (segment (start 116.125095 70.948064) (end 125.200219 80.023188) (width 0.2) (layer "F.Cu") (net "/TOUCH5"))
 (segment (start 96.931564 70.948064) (end 116.125095 70.948064) (width 0.2) (layer "F.Cu") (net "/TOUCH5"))
 (segment (start 92.6035 66.62) (end 96.931564 70.948064) (width 0.2) (layer "F.Cu") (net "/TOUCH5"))
 (segment (start 125.200219 80.023188) (end 125.200219 130.799781) (width 0.2) (layer "F.Cu") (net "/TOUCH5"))
 (segment (start 99.071564 70.548064) (end 122.548064 70.548064) (width 0.2) (layer "F.Cu") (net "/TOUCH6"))
 (segment (start 95.1435 66.62) (end 99.071564 70.548064) (width 0.2) (layer "F.Cu") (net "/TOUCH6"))
 (segment (start 122.548064 70.548064) (end 141 89) (width 0.2) (layer "F.Cu") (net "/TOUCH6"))
 (segment (start 101.4035 62.9) (end 97.6835 66.62) (width 0.2) (layer "B.Cu") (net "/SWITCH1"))
 (segment (start 109 62.9) (end 101.4035 62.9) (width 0.2) (layer "B.Cu") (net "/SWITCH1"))
 (segment (start 66.54 59.46) (end 72.872918 59.46) (width 0.2) (layer "F.Cu") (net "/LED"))
 (segment (start 61.275 64.725) (end 66.54 59.46) (width 0.2) (layer "F.Cu") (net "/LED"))
 (segment (start 91.5495 50.326) (end 92.6035 51.38) (width 0.2) (layer "F.Cu") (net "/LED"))
 (segment (start 61.275 65.25) (end 61.275 64.725) (width 0.2) (layer "F.Cu") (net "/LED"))
 (segment (start 72.872918 59.46) (end 82.006918 50.326) (width 0.2) (layer "F.Cu") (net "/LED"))
 (segment (start 82.006918 50.326) (end 91.5495 50.326) (width 0.2) (layer "F.Cu") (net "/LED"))
 (segment (start 104.9995 66.316) (end 90.0635 51.38) (width 0.2) (layer "F.Cu") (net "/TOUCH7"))
 (segment (start 157 83.802194) (end 139.513806 66.316) (width 0.2) (layer "F.Cu") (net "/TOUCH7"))
 (segment (start 157 129) (end 157 83.802194) (width 0.2) (layer "F.Cu") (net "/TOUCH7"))
 (segment (start 139.513806 66.316) (end 104.9995 66.316) (width 0.2) (layer "F.Cu") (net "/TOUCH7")))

